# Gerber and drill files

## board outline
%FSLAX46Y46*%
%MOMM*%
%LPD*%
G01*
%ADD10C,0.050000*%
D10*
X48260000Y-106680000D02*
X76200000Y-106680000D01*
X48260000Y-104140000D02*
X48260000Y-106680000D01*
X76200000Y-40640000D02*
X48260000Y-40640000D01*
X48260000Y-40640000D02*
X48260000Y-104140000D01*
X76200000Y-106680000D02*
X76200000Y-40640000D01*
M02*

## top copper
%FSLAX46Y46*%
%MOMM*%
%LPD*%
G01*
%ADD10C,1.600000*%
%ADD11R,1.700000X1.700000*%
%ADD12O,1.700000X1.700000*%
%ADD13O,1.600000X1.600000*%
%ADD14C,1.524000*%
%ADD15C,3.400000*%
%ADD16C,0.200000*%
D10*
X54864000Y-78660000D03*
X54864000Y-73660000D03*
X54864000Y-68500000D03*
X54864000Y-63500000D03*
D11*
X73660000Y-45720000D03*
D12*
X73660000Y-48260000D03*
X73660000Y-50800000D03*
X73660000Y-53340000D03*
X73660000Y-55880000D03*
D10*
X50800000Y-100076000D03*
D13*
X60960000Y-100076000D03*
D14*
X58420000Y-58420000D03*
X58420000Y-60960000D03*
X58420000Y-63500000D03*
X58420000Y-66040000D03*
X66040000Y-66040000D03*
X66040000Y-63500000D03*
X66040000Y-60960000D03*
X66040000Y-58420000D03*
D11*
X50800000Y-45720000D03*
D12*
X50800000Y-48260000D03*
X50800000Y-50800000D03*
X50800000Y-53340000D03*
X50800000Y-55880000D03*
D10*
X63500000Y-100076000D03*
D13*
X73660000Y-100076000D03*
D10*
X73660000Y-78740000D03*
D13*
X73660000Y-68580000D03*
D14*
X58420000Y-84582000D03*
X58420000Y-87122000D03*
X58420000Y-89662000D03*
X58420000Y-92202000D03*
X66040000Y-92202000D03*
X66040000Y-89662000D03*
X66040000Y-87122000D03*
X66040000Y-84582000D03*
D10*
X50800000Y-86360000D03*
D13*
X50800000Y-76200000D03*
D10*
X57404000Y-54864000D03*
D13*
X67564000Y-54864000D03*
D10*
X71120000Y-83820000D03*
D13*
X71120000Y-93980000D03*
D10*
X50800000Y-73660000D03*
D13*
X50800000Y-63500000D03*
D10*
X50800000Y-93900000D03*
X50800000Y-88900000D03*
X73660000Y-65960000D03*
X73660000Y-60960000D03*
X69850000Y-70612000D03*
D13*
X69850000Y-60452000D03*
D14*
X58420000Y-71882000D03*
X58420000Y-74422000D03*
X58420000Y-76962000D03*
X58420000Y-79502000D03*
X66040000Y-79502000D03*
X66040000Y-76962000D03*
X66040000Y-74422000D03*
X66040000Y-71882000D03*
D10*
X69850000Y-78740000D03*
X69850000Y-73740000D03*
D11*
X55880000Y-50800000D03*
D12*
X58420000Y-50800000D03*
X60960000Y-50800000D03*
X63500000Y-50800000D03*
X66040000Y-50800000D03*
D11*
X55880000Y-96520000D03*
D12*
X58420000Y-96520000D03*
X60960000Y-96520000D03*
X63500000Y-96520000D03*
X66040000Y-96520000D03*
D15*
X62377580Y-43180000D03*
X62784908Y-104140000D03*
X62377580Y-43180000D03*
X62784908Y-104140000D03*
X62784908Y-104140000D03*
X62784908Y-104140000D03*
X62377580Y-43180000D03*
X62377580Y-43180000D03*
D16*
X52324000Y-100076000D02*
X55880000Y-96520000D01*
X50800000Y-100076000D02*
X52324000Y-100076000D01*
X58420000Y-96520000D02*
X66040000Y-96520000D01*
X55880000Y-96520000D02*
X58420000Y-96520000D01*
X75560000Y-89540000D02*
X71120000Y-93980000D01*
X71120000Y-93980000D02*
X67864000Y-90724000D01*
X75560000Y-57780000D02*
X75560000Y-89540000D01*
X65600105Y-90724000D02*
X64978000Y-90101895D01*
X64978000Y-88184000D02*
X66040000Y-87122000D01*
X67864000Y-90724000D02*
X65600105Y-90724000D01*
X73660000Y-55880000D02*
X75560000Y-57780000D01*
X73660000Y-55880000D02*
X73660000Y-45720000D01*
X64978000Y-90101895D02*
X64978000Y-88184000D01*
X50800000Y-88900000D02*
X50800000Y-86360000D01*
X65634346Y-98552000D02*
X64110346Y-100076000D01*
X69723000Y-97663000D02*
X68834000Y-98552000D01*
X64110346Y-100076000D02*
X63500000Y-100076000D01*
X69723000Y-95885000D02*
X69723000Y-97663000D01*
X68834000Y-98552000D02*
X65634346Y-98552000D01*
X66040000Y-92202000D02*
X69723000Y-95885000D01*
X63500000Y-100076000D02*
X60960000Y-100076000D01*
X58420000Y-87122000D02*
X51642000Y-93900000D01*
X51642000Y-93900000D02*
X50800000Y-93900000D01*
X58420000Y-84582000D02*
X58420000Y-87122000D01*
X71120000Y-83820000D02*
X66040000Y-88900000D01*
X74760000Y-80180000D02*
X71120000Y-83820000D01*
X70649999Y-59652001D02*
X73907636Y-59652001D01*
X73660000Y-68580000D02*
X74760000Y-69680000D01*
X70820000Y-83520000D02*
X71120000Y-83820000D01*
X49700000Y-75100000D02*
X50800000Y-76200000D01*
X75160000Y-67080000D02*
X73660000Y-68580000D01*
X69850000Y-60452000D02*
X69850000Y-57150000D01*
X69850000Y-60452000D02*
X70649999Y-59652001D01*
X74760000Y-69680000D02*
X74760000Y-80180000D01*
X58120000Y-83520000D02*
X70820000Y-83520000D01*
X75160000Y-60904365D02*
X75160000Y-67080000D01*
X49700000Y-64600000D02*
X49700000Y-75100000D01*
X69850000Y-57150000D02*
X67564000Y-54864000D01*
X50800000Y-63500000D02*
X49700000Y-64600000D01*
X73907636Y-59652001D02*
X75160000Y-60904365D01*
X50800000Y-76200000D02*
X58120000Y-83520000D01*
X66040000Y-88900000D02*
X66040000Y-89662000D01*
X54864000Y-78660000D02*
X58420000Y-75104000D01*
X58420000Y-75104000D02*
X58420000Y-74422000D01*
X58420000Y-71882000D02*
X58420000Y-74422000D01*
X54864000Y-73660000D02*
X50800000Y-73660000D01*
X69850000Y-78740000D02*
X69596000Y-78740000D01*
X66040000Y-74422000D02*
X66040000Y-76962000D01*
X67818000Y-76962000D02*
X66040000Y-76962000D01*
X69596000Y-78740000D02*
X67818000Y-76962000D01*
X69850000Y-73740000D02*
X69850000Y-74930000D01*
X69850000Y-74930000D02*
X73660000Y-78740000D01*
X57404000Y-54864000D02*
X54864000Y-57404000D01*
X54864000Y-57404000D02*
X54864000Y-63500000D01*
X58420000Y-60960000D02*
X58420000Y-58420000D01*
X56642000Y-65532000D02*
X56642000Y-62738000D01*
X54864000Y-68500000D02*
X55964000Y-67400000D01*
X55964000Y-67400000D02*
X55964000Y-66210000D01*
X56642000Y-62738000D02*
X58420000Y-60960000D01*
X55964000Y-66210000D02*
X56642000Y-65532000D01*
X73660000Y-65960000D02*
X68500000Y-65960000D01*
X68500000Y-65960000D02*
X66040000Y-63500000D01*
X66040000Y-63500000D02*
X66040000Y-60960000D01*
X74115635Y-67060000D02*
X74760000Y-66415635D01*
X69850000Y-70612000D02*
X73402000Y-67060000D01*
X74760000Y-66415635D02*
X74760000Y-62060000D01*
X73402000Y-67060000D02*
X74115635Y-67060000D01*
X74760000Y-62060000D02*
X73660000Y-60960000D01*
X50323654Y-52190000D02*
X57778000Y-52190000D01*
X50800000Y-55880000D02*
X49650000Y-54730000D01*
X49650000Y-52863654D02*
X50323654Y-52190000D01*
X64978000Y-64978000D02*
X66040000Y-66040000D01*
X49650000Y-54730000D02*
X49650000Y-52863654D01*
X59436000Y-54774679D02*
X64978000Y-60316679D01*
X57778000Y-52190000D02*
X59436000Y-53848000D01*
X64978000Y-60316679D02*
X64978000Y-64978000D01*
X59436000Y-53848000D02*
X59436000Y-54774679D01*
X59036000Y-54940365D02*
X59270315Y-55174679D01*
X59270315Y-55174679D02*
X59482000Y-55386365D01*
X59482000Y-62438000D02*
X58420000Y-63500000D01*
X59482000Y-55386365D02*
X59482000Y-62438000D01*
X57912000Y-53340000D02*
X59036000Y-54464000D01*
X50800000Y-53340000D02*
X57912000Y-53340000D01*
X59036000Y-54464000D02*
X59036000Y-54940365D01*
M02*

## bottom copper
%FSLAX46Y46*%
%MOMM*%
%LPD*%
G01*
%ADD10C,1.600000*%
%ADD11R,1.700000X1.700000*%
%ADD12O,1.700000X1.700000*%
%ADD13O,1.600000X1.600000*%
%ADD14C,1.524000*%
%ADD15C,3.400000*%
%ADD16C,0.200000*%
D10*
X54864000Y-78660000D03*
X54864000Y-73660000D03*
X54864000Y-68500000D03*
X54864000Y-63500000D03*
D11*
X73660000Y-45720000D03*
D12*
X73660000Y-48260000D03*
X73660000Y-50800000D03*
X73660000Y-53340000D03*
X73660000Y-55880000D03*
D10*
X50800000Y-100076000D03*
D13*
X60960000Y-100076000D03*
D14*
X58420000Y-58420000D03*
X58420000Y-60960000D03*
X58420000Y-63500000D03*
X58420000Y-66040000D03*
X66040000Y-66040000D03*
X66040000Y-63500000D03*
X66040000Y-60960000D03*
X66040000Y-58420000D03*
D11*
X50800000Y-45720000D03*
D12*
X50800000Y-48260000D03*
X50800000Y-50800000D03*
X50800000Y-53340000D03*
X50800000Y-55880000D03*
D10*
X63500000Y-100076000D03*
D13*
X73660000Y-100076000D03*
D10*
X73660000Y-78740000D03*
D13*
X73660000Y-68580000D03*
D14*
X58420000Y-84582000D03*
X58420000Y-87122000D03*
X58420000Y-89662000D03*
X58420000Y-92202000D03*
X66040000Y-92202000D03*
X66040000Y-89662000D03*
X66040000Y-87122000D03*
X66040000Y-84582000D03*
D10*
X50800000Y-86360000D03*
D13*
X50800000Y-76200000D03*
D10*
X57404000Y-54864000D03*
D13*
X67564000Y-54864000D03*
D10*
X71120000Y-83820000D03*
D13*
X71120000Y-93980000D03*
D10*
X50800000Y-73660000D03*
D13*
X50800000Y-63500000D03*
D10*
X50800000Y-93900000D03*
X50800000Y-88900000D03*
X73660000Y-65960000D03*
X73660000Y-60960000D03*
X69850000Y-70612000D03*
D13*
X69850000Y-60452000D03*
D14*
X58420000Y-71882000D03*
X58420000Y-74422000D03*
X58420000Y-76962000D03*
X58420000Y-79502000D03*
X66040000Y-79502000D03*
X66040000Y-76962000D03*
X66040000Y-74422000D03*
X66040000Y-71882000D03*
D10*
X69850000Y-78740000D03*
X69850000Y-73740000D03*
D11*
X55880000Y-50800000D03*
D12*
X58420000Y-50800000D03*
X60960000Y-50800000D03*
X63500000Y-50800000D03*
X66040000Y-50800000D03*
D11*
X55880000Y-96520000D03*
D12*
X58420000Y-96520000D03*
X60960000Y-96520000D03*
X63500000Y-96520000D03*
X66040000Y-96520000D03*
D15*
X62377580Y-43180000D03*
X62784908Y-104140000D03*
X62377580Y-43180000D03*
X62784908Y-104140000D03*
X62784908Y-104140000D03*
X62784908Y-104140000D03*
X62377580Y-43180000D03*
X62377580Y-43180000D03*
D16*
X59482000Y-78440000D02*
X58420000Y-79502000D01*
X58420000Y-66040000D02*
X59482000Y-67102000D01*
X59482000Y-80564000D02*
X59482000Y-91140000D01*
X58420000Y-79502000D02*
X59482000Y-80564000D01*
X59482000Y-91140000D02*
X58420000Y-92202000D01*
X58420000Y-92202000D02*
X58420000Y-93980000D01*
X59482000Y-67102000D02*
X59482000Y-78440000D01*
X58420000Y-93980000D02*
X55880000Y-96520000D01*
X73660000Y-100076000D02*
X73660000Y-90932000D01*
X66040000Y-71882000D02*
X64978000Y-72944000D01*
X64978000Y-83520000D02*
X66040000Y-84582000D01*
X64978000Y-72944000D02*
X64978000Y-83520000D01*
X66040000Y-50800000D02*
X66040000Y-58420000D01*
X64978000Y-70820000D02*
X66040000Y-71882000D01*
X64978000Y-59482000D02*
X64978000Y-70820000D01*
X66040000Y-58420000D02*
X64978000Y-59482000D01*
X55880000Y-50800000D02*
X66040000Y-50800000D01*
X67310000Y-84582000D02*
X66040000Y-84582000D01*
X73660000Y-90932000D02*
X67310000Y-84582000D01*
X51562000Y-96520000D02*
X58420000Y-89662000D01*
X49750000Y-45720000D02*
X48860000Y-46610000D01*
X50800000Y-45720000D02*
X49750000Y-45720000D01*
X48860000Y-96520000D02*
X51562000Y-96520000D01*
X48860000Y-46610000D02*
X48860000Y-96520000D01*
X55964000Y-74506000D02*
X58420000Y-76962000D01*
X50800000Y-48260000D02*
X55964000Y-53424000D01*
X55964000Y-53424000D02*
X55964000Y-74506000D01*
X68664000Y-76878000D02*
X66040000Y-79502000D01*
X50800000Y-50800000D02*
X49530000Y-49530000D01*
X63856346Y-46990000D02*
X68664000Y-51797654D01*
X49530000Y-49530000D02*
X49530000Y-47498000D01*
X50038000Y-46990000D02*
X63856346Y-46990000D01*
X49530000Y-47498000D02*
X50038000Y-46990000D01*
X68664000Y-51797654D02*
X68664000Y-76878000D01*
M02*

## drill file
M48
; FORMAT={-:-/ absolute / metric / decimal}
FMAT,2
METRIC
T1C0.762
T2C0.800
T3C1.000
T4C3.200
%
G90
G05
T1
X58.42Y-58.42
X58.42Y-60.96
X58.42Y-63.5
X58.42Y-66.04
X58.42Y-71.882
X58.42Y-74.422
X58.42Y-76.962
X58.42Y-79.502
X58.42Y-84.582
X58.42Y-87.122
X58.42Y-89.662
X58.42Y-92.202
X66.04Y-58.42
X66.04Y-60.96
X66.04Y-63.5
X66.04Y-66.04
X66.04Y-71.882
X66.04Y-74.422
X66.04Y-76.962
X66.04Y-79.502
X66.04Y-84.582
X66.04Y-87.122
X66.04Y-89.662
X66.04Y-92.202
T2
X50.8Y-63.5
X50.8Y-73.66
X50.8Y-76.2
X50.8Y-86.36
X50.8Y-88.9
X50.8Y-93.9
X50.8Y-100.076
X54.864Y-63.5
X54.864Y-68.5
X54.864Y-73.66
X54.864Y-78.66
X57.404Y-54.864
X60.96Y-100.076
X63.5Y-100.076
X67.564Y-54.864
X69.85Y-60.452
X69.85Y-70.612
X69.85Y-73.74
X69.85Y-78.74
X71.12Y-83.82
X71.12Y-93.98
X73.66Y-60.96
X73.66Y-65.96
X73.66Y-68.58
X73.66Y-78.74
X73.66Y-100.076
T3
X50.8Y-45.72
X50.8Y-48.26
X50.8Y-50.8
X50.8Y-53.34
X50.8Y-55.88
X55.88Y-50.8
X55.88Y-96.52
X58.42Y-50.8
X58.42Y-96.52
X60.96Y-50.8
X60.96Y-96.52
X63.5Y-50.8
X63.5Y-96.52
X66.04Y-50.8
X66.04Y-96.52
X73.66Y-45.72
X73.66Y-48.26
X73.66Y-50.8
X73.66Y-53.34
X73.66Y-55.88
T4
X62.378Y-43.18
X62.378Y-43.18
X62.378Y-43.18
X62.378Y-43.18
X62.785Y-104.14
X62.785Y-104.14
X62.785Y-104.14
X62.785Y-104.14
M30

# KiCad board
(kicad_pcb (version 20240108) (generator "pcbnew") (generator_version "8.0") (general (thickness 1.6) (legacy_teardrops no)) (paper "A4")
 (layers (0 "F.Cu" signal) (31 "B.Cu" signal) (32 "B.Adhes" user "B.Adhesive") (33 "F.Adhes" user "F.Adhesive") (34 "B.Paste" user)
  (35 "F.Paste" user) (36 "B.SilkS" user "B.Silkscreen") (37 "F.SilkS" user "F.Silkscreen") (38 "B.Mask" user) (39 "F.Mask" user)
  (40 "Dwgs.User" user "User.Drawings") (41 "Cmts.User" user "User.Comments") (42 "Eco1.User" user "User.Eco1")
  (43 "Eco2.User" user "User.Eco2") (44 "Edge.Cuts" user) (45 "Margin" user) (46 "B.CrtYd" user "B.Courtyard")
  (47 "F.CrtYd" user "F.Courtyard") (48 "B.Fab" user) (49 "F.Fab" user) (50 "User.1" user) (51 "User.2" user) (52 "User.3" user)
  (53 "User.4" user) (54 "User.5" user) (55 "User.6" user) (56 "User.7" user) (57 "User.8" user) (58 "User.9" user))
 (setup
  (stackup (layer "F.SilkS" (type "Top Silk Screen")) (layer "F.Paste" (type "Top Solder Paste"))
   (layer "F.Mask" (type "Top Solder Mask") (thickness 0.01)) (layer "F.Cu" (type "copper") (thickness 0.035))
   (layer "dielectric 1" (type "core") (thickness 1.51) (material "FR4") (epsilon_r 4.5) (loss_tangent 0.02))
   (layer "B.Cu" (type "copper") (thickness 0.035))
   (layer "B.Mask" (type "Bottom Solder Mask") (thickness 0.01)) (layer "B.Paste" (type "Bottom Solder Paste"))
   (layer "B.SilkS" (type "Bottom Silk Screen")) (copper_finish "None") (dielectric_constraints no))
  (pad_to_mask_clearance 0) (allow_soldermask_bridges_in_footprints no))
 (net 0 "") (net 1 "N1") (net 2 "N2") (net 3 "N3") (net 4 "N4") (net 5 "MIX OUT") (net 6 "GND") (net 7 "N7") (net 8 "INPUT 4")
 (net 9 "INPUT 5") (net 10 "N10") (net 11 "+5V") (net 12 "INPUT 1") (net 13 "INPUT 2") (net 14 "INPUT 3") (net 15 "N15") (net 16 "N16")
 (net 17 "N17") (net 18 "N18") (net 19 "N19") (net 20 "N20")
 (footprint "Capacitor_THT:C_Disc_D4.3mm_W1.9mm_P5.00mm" (layer "F.Cu") (at 54.864 78.66 90)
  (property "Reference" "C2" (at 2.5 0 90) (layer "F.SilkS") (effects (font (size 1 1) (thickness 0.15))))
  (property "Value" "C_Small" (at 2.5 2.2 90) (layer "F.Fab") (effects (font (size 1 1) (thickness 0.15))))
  (pad "1" thru_hole circle (at 0 0 90) (size 1.6 1.6) (drill 0.8) (layers "*.Cu" "*.Mask") (remove_unused_layers no) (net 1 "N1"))
  (pad "2" thru_hole circle (at 5 0 90) (size 1.6 1.6) (drill 0.8) (layers "*.Cu" "*.Mask") (remove_unused_layers no) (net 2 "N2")))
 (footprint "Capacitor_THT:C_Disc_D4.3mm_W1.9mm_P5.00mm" (layer "F.Cu") (at 54.864 68.5 90)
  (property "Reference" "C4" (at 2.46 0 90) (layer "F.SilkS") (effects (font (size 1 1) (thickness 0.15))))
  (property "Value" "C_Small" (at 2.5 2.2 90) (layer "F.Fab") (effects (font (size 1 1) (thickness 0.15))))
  (pad "1" thru_hole circle (at 0 0 90) (size 1.6 1.6) (drill 0.8) (layers "*.Cu" "*.Mask") (remove_unused_layers no) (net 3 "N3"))
  (pad "2" thru_hole circle (at 5 0 90) (size 1.6 1.6) (drill 0.8) (layers "*.Cu" "*.Mask") (remove_unused_layers no) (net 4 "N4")))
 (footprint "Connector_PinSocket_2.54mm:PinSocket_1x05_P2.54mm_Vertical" (layer "F.Cu") (at 73.66 45.72)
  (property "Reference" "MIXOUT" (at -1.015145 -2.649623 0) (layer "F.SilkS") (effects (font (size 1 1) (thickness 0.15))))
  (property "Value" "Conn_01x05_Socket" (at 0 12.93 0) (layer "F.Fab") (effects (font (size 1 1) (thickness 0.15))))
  (pad "1" thru_hole rect (at 0 0) (size 1.7 1.7) (drill 1) (layers "*.Cu" "*.Mask") (remove_unused_layers no) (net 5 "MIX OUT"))
  (pad "2" thru_hole oval (at 0 2.54) (size 1.7 1.7) (drill 1) (layers "*.Cu" "*.Mask") (remove_unused_layers no) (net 5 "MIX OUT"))
  (pad "3" thru_hole oval (at 0 5.08) (size 1.7 1.7) (drill 1) (layers "*.Cu" "*.Mask") (remove_unused_layers no) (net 5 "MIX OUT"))
  (pad "4" thru_hole oval (at 0 7.62) (size 1.7 1.7) (drill 1) (layers "*.Cu" "*.Mask") (remove_unused_layers no) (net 5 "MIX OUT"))
  (pad "5" thru_hole oval (at 0 10.16) (size 1.7 1.7) (drill 1) (layers "*.Cu" "*.Mask") (remove_unused_layers no) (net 5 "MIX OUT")))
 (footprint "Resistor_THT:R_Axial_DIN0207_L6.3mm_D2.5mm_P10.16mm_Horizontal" (layer "F.Cu") (at 50.8 100.076)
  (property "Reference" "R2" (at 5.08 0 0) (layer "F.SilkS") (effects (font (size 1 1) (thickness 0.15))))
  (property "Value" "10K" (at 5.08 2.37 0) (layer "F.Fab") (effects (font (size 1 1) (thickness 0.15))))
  (pad "1" thru_hole circle (at 0 0) (size 1.6 1.6) (drill 0.8) (layers "*.Cu" "*.Mask") (remove_unused_layers no) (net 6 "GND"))
  (pad "2" thru_hole oval (at 10.16 0) (size 1.6 1.6) (drill 0.8) (layers "*.Cu" "*.Mask") (remove_unused_layers no) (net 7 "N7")))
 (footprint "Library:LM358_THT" (layer "F.Cu") (at 61.214 62.738 -90)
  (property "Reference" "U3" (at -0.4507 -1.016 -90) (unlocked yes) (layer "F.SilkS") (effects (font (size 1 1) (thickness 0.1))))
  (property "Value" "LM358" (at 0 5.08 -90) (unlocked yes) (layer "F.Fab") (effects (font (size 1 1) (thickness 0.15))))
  (pad "1" thru_hole circle (at -4.318 2.794 270) (size 1.524 1.524) (drill 0.762) (layers "*.Cu" "*.Mask") (remove_unused_layers no)
   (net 3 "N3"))
  (pad "2" thru_hole circle (at -1.778 2.794 270) (size 1.524 1.524) (drill 0.762) (layers "*.Cu" "*.Mask") (remove_unused_layers no)
   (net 3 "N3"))
  (pad "3" thru_hole circle (at 0.762 2.794 270) (size 1.524 1.524) (drill 0.762) (layers "*.Cu" "*.Mask") (remove_unused_layers no)
   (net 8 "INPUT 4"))
  (pad "4" thru_hole circle (at 3.302 2.794 270) (size 1.524 1.524) (drill 0.762) (layers "*.Cu" "*.Mask") (remove_unused_layers no)
   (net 6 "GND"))
  (pad "5" thru_hole circle (at 3.302 -4.826 270) (size 1.524 1.524) (drill 0.762) (layers "*.Cu" "*.Mask") (remove_unused_layers no)
   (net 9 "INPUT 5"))
  (pad "6" thru_hole circle (at 0.762 -4.826 270) (size 1.524 1.524) (drill 0.762) (layers "*.Cu" "*.Mask") (remove_unused_layers no)
   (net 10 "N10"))
  (pad "7" thru_hole circle (at -1.778 -4.826 270) (size 1.524 1.524) (drill 0.762) (layers "*.Cu" "*.Mask") (remove_unused_layers no)
   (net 10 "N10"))
  (pad "8" thru_hole circle (at -4.318 -4.826 270) (size 1.524 1.524) (drill 0.762) (layers "*.Cu" "*.Mask") (remove_unused_layers no)
   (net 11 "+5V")))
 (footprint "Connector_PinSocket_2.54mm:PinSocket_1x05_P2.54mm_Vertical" (layer "F.Cu") (at 50.8 45.72)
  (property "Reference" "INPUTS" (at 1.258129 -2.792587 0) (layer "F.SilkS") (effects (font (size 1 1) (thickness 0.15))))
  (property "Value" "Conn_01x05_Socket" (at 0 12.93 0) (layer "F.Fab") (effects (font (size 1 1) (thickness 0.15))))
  (pad "1" thru_hole rect (at 0 0) (size 1.7 1.7) (drill 1) (layers "*.Cu" "*.Mask") (remove_unused_layers no) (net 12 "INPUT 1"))
  (pad "2" thru_hole oval (at 0 2.54) (size 1.7 1.7) (drill 1) (layers "*.Cu" "*.Mask") (remove_unused_layers no) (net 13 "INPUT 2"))
  (pad "3" thru_hole oval (at 0 5.08) (size 1.7 1.7) (drill 1) (layers "*.Cu" "*.Mask") (remove_unused_layers no) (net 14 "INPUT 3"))
  (pad "4" thru_hole oval (at 0 7.62) (size 1.7 1.7) (drill 1) (layers "*.Cu" "*.Mask") (remove_unused_layers no) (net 8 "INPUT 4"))
  (pad "5" thru_hole oval (at 0 10.16) (size 1.7 1.7) (drill 1) (layers "*.Cu" "*.Mask") (remove_unused_layers no) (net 9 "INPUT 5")))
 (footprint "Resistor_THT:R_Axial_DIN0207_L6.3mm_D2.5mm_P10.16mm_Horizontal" (layer "F.Cu") (at 63.5 100.076)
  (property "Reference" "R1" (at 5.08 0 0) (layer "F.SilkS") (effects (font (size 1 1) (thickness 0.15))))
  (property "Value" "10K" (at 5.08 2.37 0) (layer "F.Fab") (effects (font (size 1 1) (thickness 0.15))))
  (pad "1" thru_hole circle (at 0 0) (size 1.6 1.6) (drill 0.8) (layers "*.Cu" "*.Mask") (remove_unused_layers no) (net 7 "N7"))
  (pad "2" thru_hole oval (at 10.16 0) (size 1.6 1.6) (drill 0.8) (layers "*.Cu" "*.Mask") (remove_unused_layers no) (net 11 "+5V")))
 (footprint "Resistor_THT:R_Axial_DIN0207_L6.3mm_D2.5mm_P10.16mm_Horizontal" (layer "F.Cu") (at 73.66 78.74 90)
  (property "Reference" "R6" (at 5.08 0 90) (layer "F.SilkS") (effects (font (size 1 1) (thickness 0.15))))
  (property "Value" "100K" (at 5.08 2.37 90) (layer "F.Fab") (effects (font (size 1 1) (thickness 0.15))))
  (pad "1" thru_hole circle (at 0 0 90) (size 1.6 1.6) (drill 0.8) (layers "*.Cu" "*.Mask") (remove_unused_layers no) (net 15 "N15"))
  (pad "2" thru_hole oval (at 10.16 0 90) (size 1.6 1.6) (drill 0.8) (layers "*.Cu" "*.Mask") (remove_unused_layers no) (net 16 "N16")))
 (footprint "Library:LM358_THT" (layer "F.Cu") (at 61.214 88.9 -90)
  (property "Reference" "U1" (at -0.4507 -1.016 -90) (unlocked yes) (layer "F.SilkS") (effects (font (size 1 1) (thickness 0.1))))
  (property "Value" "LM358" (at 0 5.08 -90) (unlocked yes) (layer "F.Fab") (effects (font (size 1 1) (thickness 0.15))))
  (pad "1" thru_hole circle (at -4.318 2.794 270) (size 1.524 1.524) (drill 0.762) (layers "*.Cu" "*.Mask") (remove_unused_layers no)
   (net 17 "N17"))
  (pad "2" thru_hole circle (at -1.778 2.794 270) (size 1.524 1.524) (drill 0.762) (layers "*.Cu" "*.Mask") (remove_unused_layers no)
   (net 17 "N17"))
  (pad "3" thru_hole circle (at 0.762 2.794 270) (size 1.524 1.524) (drill 0.762) (layers "*.Cu" "*.Mask") (remove_unused_layers no)
   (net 12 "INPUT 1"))
  (pad "4" thru_hole circle (at 3.302 2.794 270) (size 1.524 1.524) (drill 0.762) (layers "*.Cu" "*.Mask") (remove_unused_layers no)
   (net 6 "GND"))
  (pad "5" thru_hole circle (at 3.302 -4.826 270) (size 1.524 1.524) (drill 0.762) (layers "*.Cu" "*.Mask") (remove_unused_layers no)
   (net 7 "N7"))
  (pad "6" thru_hole circle (at 0.762 -4.826 270) (size 1.524 1.524) (drill 0.762) (layers "*.Cu" "*.Mask") (remove_unused_layers no)
   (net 16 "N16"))
  (pad "7" thru_hole circle (at -1.778 -4.826 270) (size 1.524 1.524) (drill 0.762) (layers "*.Cu" "*.Mask") (remove_unused_layers no)
   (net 5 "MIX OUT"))
  (pad "8" thru_hole circle (at -4.318 -4.826 270) (size 1.524 1.524) (drill 0.762) (layers "*.Cu" "*.Mask") (remove_unused_layers no)
   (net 11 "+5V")))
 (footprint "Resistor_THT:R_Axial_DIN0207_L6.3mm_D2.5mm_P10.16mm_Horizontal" (layer "F.Cu") (at 50.8 86.36 90)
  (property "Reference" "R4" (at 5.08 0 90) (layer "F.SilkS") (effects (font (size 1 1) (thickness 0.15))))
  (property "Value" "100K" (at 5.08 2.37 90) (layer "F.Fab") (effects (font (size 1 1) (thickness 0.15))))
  (pad "1" thru_hole circle (at 0 0 90) (size 1.6 1.6) (drill 0.8) (layers "*.Cu" "*.Mask") (remove_unused_layers no) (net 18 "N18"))
  (pad "2" thru_hole oval (at 10.16 0 90) (size 1.6 1.6) (drill 0.8) (layers "*.Cu" "*.Mask") (remove_unused_layers no) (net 16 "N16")))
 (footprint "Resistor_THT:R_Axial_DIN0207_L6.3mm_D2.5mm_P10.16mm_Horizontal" (layer "F.Cu") (at 57.404 54.864)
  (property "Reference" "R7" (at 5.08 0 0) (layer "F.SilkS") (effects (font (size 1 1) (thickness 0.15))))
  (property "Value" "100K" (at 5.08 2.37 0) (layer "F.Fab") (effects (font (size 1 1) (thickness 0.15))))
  (pad "1" thru_hole circle (at 0 0) (size 1.6 1.6) (drill 0.8) (layers "*.Cu" "*.Mask") (remove_unused_layers no) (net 4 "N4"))
  (pad "2" thru_hole oval (at 10.16 0) (size 1.6 1.6) (drill 0.8) (layers "*.Cu" "*.Mask") (remove_unused_layers no) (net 16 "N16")))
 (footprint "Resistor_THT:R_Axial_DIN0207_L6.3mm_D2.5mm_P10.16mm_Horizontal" (layer "F.Cu") (at 71.12 83.82 -90)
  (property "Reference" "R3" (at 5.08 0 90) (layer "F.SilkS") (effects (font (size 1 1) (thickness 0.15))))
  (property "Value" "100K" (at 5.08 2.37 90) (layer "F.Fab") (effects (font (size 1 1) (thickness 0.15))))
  (pad "1" thru_hole circle (at 0 0 270) (size 1.6 1.6) (drill 0.8) (layers "*.Cu" "*.Mask") (remove_unused_layers no) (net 16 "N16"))
  (pad "2" thru_hole oval (at 10.16 0 270) (size 1.6 1.6) (drill 0.8) (layers "*.Cu" "*.Mask") (remove_unused_layers no) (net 5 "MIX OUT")))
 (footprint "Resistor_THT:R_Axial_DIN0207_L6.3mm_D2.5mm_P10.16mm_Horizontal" (layer "F.Cu") (at 50.8 73.66 90)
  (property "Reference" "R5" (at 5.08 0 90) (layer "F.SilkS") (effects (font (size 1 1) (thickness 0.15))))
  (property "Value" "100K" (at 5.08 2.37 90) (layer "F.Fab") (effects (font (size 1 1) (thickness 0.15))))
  (pad "1" thru_hole circle (at 0 0 90) (size 1.6 1.6) (drill 0.8) (layers "*.Cu" "*.Mask") (remove_unused_layers no) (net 2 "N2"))
  (pad "2" thru_hole oval (at 10.16 0 90) (size 1.6 1.6) (drill 0.8) (layers "*.Cu" "*.Mask") (remove_unused_layers no) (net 16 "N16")))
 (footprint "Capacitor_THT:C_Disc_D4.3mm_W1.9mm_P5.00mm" (layer "F.Cu") (at 50.8 93.9 90)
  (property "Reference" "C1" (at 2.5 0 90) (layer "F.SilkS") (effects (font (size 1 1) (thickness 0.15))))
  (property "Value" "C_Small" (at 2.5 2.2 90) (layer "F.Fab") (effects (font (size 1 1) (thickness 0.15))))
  (pad "1" thru_hole circle (at 0 0 90) (size 1.6 1.6) (drill 0.8) (layers "*.Cu" "*.Mask") (remove_unused_layers no) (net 17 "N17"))
  (pad "2" thru_hole circle (at 5 0 90) (size 1.6 1.6) (drill 0.8) (layers "*.Cu" "*.Mask") (remove_unused_layers no) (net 18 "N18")))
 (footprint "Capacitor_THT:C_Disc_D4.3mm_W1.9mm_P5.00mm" (layer "F.Cu") (at 73.66 65.96 90)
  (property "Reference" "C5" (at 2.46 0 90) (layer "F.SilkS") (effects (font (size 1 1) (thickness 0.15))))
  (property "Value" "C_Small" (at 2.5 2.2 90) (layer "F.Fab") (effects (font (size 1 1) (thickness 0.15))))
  (pad "1" thru_hole circle (at 0 0 90) (size 1.6 1.6) (drill 0.8) (layers "*.Cu" "*.Mask") (remove_unused_layers no) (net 10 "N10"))
  (pad "2" thru_hole circle (at 5 0 90) (size 1.6 1.6) (drill 0.8) (layers "*.Cu" "*.Mask") (remove_unused_layers no) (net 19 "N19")))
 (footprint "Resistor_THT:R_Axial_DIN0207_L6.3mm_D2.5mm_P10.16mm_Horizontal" (layer "F.Cu") (at 69.85 70.612 90)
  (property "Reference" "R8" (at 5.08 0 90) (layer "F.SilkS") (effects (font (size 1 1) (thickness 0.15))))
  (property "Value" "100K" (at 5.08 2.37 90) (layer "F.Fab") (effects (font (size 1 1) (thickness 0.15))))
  (pad "1" thru_hole circle (at 0 0 90) (size 1.6 1.6) (drill 0.8) (layers "*.Cu" "*.Mask") (remove_unused_layers no) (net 19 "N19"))
  (pad "2" thru_hole oval (at 10.16 0 90) (size 1.6 1.6) (drill 0.8) (layers "*.Cu" "*.Mask") (remove_unused_layers no) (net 16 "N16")))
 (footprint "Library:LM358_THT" (layer "F.Cu") (at 61.214 76.2 -90)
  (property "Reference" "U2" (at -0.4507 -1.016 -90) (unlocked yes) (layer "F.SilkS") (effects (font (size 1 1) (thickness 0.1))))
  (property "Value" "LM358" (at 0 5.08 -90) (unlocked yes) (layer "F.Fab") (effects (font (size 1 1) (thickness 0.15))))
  (pad "1" thru_hole circle (at -4.318 2.794 270) (size 1.524 1.524) (drill 0.762) (layers "*.Cu" "*.Mask") (remove_unused_layers no)
   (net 1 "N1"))
  (pad "2" thru_hole circle (at -1.778 2.794 270) (size 1.524 1.524) (drill 0.762) (layers "*.Cu" "*.Mask") (remove_unused_layers no)
   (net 1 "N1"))
  (pad "3" thru_hole circle (at 0.762 2.794 270) (size 1.524 1.524) (drill 0.762) (layers "*.Cu" "*.Mask") (remove_unused_layers no)
   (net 13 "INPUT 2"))
  (pad "4" thru_hole circle (at 3.302 2.794 270) (size 1.524 1.524) (drill 0.762) (layers "*.Cu" "*.Mask") (remove_unused_layers no)
   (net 6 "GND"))
  (pad "5" thru_hole circle (at 3.302 -4.826 270) (size 1.524 1.524) (drill 0.762) (layers "*.Cu" "*.Mask") (remove_unused_layers no)
   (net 14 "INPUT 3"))
  (pad "6" thru_hole circle (at 0.762 -4.826 270) (size 1.524 1.524) (drill 0.762) (layers "*.Cu" "*.Mask") (remove_unused_layers no)
   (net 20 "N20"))
  (pad "7" thru_hole circle (at -1.778 -4.826 270) (size 1.524 1.524) (drill 0.762) (layers "*.Cu" "*.Mask") (remove_unused_layers no)
   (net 20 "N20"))
  (pad "8" thru_hole circle (at -4.318 -4.826 270) (size 1.524 1.524) (drill 0.762) (layers "*.Cu" "*.Mask") (remove_unused_layers no)
   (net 11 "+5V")))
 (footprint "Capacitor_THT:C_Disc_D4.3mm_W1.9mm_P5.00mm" (layer "F.Cu") (at 69.85 78.74 90)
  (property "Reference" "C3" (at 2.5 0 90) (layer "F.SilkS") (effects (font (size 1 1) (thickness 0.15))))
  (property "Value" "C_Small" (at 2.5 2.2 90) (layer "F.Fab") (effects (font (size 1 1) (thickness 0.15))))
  (pad "1" thru_hole circle (at 0 0 90) (size 1.6 1.6) (drill 0.8) (layers "*.Cu" "*.Mask") (remove_unused_layers no) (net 20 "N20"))
  (pad "2" thru_hole circle (at 5 0 90) (size 1.6 1.6) (drill 0.8) (layers "*.Cu" "*.Mask") (remove_unused_layers no) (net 15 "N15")))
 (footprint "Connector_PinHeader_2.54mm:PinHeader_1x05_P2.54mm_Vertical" (layer "B.Cu") (at 55.88 50.8 -90)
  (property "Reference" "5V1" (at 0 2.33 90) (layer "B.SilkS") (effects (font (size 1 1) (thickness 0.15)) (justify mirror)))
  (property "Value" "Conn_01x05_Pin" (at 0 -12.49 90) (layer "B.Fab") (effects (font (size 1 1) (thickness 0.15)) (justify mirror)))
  (pad "1" thru_hole rect (at 0 0 270) (size 1.7 1.7) (drill 1) (layers "*.Cu" "*.Mask") (remove_unused_layers no) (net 11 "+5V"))
  (pad "2" thru_hole oval (at 0 -2.54 270) (size 1.7 1.7) (drill 1) (layers "*.Cu" "*.Mask") (remove_unused_layers no) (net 11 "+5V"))
  (pad "3" thru_hole oval (at 0 -5.08 270) (size 1.7 1.7) (drill 1) (layers "*.Cu" "*.Mask") (remove_unused_layers no) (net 11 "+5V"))
  (pad "4" thru_hole oval (at 0 -7.62 270) (size 1.7 1.7) (drill 1) (layers "*.Cu" "*.Mask") (remove_unused_layers no) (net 11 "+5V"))
  (pad "5" thru_hole oval (at 0 -10.16 270) (size 1.7 1.7) (drill 1) (layers "*.Cu" "*.Mask") (remove_unused_layers no) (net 11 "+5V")))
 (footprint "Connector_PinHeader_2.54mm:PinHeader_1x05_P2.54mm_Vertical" (layer "B.Cu") (at 55.88 96.52 -90)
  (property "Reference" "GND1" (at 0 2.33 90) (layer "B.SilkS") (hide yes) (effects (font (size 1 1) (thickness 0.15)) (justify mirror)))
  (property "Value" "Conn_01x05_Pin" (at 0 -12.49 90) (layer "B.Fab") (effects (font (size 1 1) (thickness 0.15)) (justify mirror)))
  (pad "1" thru_hole rect (at 0 0 270) (size 1.7 1.7) (drill 1) (layers "*.Cu" "*.Mask") (remove_unused_layers no) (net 6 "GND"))
  (pad "2" thru_hole oval (at 0 -2.54 270) (size 1.7 1.7) (drill 1) (layers "*.Cu" "*.Mask") (remove_unused_layers no) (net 6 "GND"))
  (pad "3" thru_hole oval (at 0 -5.08 270) (size 1.7 1.7) (drill 1) (layers "*.Cu" "*.Mask") (remove_unused_layers no) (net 6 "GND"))
  (pad "4" thru_hole oval (at 0 -7.62 270) (size 1.7 1.7) (drill 1) (layers "*.Cu" "*.Mask") (remove_unused_layers no) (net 6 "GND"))
  (pad "5" thru_hole oval (at 0 -10.16 270) (size 1.7 1.7) (drill 1) (layers "*.Cu" "*.Mask") (remove_unused_layers no) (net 6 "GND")))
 (gr_line (start 48.26 106.68) (end 76.2 106.68) (stroke (width 0.05) (type default)) (layer "Edge.Cuts"))
 (gr_line (start 48.26 104.14) (end 48.26 106.68) (stroke (width 0.05) (type default)) (layer "Edge.Cuts"))
 (gr_line (start 76.2 40.64) (end 48.26 40.64) (stroke (width 0.05) (type default)) (layer "Edge.Cuts"))
 (gr_line (start 48.26 40.64) (end 48.26 104.14) (stroke (width 0.05) (type default)) (layer "Edge.Cuts"))
 (gr_line (start 76.2 106.68) (end 76.2 40.64) (stroke (width 0.05) (type default)) (layer "Edge.Cuts"))
 (via (at 62.37758 43.18) (size 3.4) (drill 3.2) (layers "F.Cu" "B.Cu") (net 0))
 (via (at 62.784908 104.14) (size 3.4) (drill 3.2) (layers "F.Cu" "B.Cu") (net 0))
 (via (at 62.37758 43.18) (size 3.4) (drill 3.2) (layers "F.Cu" "B.Cu") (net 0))
 (via (at 62.784908 104.14) (size 3.4) (drill 3.2) (layers "F.Cu" "B.Cu") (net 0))
 (via (at 62.784908 104.14) (size 3.4) (drill 3.2) (layers "F.Cu" "B.Cu") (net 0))
 (via (at 62.784908 104.14) (size 3.4) (drill 3.2) (layers "F.Cu" "B.Cu") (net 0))
 (via (at 62.37758 43.18) (size 3.4) (drill 3.2) (layers "F.Cu" "B.Cu") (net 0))
 (via (at 62.37758 43.18) (size 3.4) (drill 3.2) (layers "F.Cu" "B.Cu") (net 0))
 (segment (start 52.324 100.076) (end 55.88 96.52) (width 0.2) (layer "F.Cu") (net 6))
 (segment (start 50.8 100.076) (end 52.324 100.076) (width 0.2) (layer "F.Cu") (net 6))
 (segment (start 58.42 96.52) (end 66.04 96.52) (width 0.2) (layer "F.Cu") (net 6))
 (segment (start 55.88 96.52) (end 58.42 96.52) (width 0.2) (layer "F.Cu") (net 6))
 (segment (start 59.482 78.44) (end 58.42 79.502) (width 0.2) (layer "B.Cu") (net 6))
 (segment (start 58.42 66.04) (end 59.482 67.102) (width 0.2) (layer "B.Cu") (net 6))
 (segment (start 59.482 80.564) (end 59.482 91.14) (width 0.2) (layer "B.Cu") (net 6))
 (segment (start 58.42 79.502) (end 59.482 80.564) (width 0.2) (layer "B.Cu") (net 6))
 (segment (start 59.482 91.14) (end 58.42 92.202) (width 0.2) (layer "B.Cu") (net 6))
 (segment (start 58.42 92.202) (end 58.42 93.98) (width 0.2) (layer "B.Cu") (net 6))
 (segment (start 59.482 67.102) (end 59.482 78.44) (width 0.2) (layer "B.Cu") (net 6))
 (segment (start 58.42 93.98) (end 55.88 96.52) (width 0.2) (layer "B.Cu") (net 6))
 (segment (start 73.66 100.076) (end 73.66 90.932) (width 0.2) (layer "B.Cu") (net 11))
 (segment (start 66.04 71.882) (end 64.978 72.944) (width 0.2) (layer "B.Cu") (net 11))
 (segment (start 64.978 83.52) (end 66.04 84.582) (width 0.2) (layer "B.Cu") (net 11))
 (segment (start 64.978 72.944) (end 64.978 83.52) (width 0.2) (layer "B.Cu") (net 11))
 (segment (start 66.04 50.8) (end 66.04 58.42) (width 0.2) (layer "B.Cu") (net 11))
 (segment (start 64.978 70.82) (end 66.04 71.882) (width 0.2) (layer "B.Cu") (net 11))
 (segment (start 64.978 59.482) (end 64.978 70.82) (width 0.2) (layer "B.Cu") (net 11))
 (segment (start 66.04 58.42) (end 64.978 59.482) (width 0.2) (layer "B.Cu") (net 11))
 (segment (start 55.88 50.8) (end 66.04 50.8) (width 0.2) (layer "B.Cu") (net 11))
 (segment (start 67.31 84.582) (end 66.04 84.582) (width 0.2) (layer "B.Cu") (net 11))
 (segment (start 73.66 90.932) (end 67.31 84.582) (width 0.2) (layer "B.Cu") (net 11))
 (segment (start 75.56 89.54) (end 71.12 93.98) (width 0.2) (layer "F.Cu") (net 5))
 (segment (start 71.12 93.98) (end 67.864 90.724) (width 0.2) (layer "F.Cu") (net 5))
 (segment (start 75.56 57.78) (end 75.56 89.54) (width 0.2) (layer "F.Cu") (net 5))
 (segment (start 65.600105 90.724) (end 64.978 90.101895) (width 0.2) (layer "F.Cu") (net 5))
 (segment (start 64.978 88.184) (end 66.04 87.122) (width 0.2) (layer "F.Cu") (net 5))
 (segment (start 67.864 90.724) (end 65.600105 90.724) (width 0.2) (layer "F.Cu") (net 5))
 (segment (start 73.66 55.88) (end 75.56 57.78) (width 0.2) (layer "F.Cu") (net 5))
 (segment (start 73.66 55.88) (end 73.66 45.72) (width 0.2) (layer "F.Cu") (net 5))
 (segment (start 64.978 90.101895) (end 64.978 88.184) (width 0.2) (layer "F.Cu") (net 5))
 (segment (start 50.8 88.9) (end 50.8 86.36) (width 0.2) (layer "F.Cu") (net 18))
 (segment (start 65.634346 98.552) (end 64.110346 100.076) (width 0.2) (layer "F.Cu") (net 7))
 (segment (start 69.723 97.663) (end 68.834 98.552) (width 0.2) (layer "F.Cu") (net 7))
 (segment (start 64.110346 100.076) (end 63.5 100.076) (width 0.2) (layer "F.Cu") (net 7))
 (segment (start 69.723 95.885) (end 69.723 97.663) (width 0.2) (layer "F.Cu") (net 7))
 (segment (start 68.834 98.552) (end 65.634346 98.552) (width 0.2) (layer "F.Cu") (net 7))
 (segment (start 66.04 92.202) (end 69.723 95.885) (width 0.2) (layer "F.Cu") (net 7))
 (segment (start 63.5 100.076) (end 60.96 100.076) (width 0.2) (layer "F.Cu") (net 7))
 (segment (start 58.42 87.122) (end 51.642 93.9) (width 0.2) (layer "F.Cu") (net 17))
 (segment (start 51.642 93.9) (end 50.8 93.9) (width 0.2) (layer "F.Cu") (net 17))
 (segment (start 58.42 84.582) (end 58.42 87.122) (width 0.2) (layer "F.Cu") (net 17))
 (segment (start 51.562 96.52) (end 58.42 89.662) (width 0.2) (layer "B.Cu") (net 12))
 (segment (start 49.75 45.72) (end 48.86 46.61) (width 0.2) (layer "B.Cu") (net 12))
 (segment (start 50.8 45.72) (end 49.75 45.72) (width 0.2) (layer "B.Cu") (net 12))
 (segment (start 48.86 96.52) (end 51.562 96.52) (width 0.2) (layer "B.Cu") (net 12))
 (segment (start 48.86 46.61) (end 48.86 96.52) (width 0.2) (layer "B.Cu") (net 12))
 (segment (start 71.12 83.82) (end 66.04 88.9) (width 0.2) (layer "F.Cu") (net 16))
 (segment (start 74.76 80.18) (end 71.12 83.82) (width 0.2) (layer "F.Cu") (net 16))
 (segment (start 70.649999 59.652001) (end 73.907636 59.652001) (width 0.2) (layer "F.Cu") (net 16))
 (segment (start 73.66 68.58) (end 74.76 69.68) (width 0.2) (layer "F.Cu") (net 16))
 (segment (start 70.82 83.52) (end 71.12 83.82) (width 0.2) (layer "F.Cu") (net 16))
 (segment (start 49.7 75.1) (end 50.8 76.2) (width 0.2) (layer "F.Cu") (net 16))
 (segment (start 75.16 67.08) (end 73.66 68.58) (width 0.2) (layer "F.Cu") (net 16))
 (segment (start 69.85 60.452) (end 69.85 57.15) (width 0.2) (layer "F.Cu") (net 16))
 (segment (start 69.85 60.452) (end 70.649999 59.652001) (width 0.2) (layer "F.Cu") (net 16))
 (segment (start 74.76 69.68) (end 74.76 80.18) (width 0.2) (layer "F.Cu") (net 16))
 (segment (start 58.12 83.52) (end 70.82 83.52) (width 0.2) (layer "F.Cu") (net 16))
 (segment (start 75.16 60.904365) (end 75.16 67.08) (width 0.2) (layer "F.Cu") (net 16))
 (segment (start 49.7 64.6) (end 49.7 75.1) (width 0.2) (layer "F.Cu") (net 16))
 (segment (start 69.85 57.15) (end 67.564 54.864) (width 0.2) (layer "F.Cu") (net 16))
 (segment (start 50.8 63.5) (end 49.7 64.6) (width 0.2) (layer "F.Cu") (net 16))
 (segment (start 73.907636 59.652001) (end 75.16 60.904365) (width 0.2) (layer "F.Cu") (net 16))
 (segment (start 50.8 76.2) (end 58.12 83.52) (width 0.2) (layer "F.Cu") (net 16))
 (segment (start 66.04 88.9) (end 66.04 89.662) (width 0.2) (layer "F.Cu") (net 16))
 (segment (start 54.864 78.66) (end 58.42 75.104) (width 0.2) (layer "F.Cu") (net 1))
 (segment (start 58.42 75.104) (end 58.42 74.422) (width 0.2) (layer "F.Cu") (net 1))
 (segment (start 58.42 71.882) (end 58.42 74.422) (width 0.2) (layer "F.Cu") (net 1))
 (segment (start 54.864 73.66) (end 50.8 73.66) (width 0.2) (layer "F.Cu") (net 2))
 (segment (start 69.85 78.74) (end 69.596 78.74) (width 0.2) (layer "F.Cu") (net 20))
 (segment (start 66.04 74.422) (end 66.04 76.962) (width 0.2) (layer "F.Cu") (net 20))
 (segment (start 67.818 76.962) (end 66.04 76.962) (width 0.2) (layer "F.Cu") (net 20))
 (segment (start 69.596 78.74) (end 67.818 76.962) (width 0.2) (layer "F.Cu") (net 20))
 (segment (start 69.85 73.74) (end 69.85 74.93) (width 0.2) (layer "F.Cu") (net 15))
 (segment (start 69.85 74.93) (end 73.66 78.74) (width 0.2) (layer "F.Cu") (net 15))
 (segment (start 57.404 54.864) (end 54.864 57.404) (width 0.2) (layer "F.Cu") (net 4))
 (segment (start 54.864 57.404) (end 54.864 63.5) (width 0.2) (layer "F.Cu") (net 4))
 (segment (start 58.42 60.96) (end 58.42 58.42) (width 0.2) (layer "F.Cu") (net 3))
 (segment (start 56.642 65.532) (end 56.642 62.738) (width 0.2) (layer "F.Cu") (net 3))
 (segment (start 54.864 68.5) (end 55.964 67.4) (width 0.2) (layer "F.Cu") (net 3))
 (segment (start 55.964 67.4) (end 55.964 66.21) (width 0.2) (layer "F.Cu") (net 3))
 (segment (start 56.642 62.738) (end 58.42 60.96) (width 0.2) (layer "F.Cu") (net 3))
 (segment (start 55.964 66.21) (end 56.642 65.532) (width 0.2) (layer "F.Cu") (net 3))
 (segment (start 73.66 65.96) (end 68.5 65.96) (width 0.2) (layer "F.Cu") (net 10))
 (segment (start 68.5 65.96) (end 66.04 63.5) (width 0.2) (layer "F.Cu") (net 10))
 (segment (start 66.04 63.5) (end 66.04 60.96) (width 0.2) (layer "F.Cu") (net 10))
 (segment (start 74.115635 67.06) (end 74.76 66.415635) (width 0.2) (layer "F.Cu") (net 19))
 (segment (start 69.85 70.612) (end 73.402 67.06) (width 0.2) (layer "F.Cu") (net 19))
 (segment (start 74.76 66.415635) (end 74.76 62.06) (width 0.2) (layer "F.Cu") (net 19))
 (segment (start 73.402 67.06) (end 74.115635 67.06) (width 0.2) (layer "F.Cu") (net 19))
 (segment (start 74.76 62.06) (end 73.66 60.96) (width 0.2) (layer "F.Cu") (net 19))
 (segment (start 50.323654 52.19) (end 57.778 52.19) (width 0.2) (layer "F.Cu") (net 9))
 (segment (start 50.8 55.88) (end 49.65 54.73) (width 0.2) (layer "F.Cu") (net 9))
 (segment (start 49.65 52.863654) (end 50.323654 52.19) (width 0.2) (layer "F.Cu") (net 9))
 (segment (start 64.978 64.978) (end 66.04 66.04) (width 0.2) (layer "F.Cu") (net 9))
 (segment (start 49.65 54.73) (end 49.65 52.863654) (width 0.2) (layer "F.Cu") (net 9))
 (segment (start 59.436 54.774679) (end 64.978 60.316679) (width 0.2) (layer "F.Cu") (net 9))
 (segment (start 57.778 52.19) (end 59.436 53.848) (width 0.2) (layer "F.Cu") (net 9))
 (segment (start 64.978 60.316679) (end 64.978 64.978) (width 0.2) (layer "F.Cu") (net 9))
 (segment (start 59.436 53.848) (end 59.436 54.774679) (width 0.2) (layer "F.Cu") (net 9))
 (segment (start 55.964 74.506) (end 58.42 76.962) (width 0.2) (layer "B.Cu") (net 13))
 (segment (start 50.8 48.26) (end 55.964 53.424) (width 0.2) (layer "B.Cu") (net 13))
 (segment (start 55.964 53.424) (end 55.964 74.506) (width 0.2) (layer "B.Cu") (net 13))
 (segment (start 59.036 54.940365) (end 59.270315 55.174679) (width 0.2) (layer "F.Cu") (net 8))
 (segment (start 59.270315 55.174679) (end 59.482 55.386365) (width 0.2) (layer "F.Cu") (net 8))
 (segment (start 59.482 62.438) (end 58.42 63.5) (width 0.2) (layer "F.Cu") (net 8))
 (segment (start 59.482 55.386365) (end 59.482 62.438) (width 0.2) (layer "F.Cu") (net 8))
 (segment (start 57.912 53.34) (end 59.036 54.464) (width 0.2) (layer "F.Cu") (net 8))
 (segment (start 50.8 53.34) (end 57.912 53.34) (width 0.2) (layer "F.Cu") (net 8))
 (segment (start 59.036 54.464) (end 59.036 54.940365) (width 0.2) (layer "F.Cu") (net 8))
 (segment (start 68.664 76.878) (end 66.04 79.502) (width 0.2) (layer "B.Cu") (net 14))
 (segment (start 50.8 50.8) (end 49.53 49.53) (width 0.2) (layer "B.Cu") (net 14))
 (segment (start 63.856346 46.99) (end 68.664 51.797654) (width 0.2) (layer "B.Cu") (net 14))
 (segment (start 49.53 49.53) (end 49.53 47.498) (width 0.2) (layer "B.Cu") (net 14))
 (segment (start 50.038 46.99) (end 63.856346 46.99) (width 0.2) (layer "B.Cu") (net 14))
 (segment (start 49.53 47.498) (end 50.038 46.99) (width 0.2) (layer "B.Cu") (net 14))
 (segment (start 68.664 51.797654) (end 68.664 76.878) (width 0.2) (layer "B.Cu") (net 14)))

